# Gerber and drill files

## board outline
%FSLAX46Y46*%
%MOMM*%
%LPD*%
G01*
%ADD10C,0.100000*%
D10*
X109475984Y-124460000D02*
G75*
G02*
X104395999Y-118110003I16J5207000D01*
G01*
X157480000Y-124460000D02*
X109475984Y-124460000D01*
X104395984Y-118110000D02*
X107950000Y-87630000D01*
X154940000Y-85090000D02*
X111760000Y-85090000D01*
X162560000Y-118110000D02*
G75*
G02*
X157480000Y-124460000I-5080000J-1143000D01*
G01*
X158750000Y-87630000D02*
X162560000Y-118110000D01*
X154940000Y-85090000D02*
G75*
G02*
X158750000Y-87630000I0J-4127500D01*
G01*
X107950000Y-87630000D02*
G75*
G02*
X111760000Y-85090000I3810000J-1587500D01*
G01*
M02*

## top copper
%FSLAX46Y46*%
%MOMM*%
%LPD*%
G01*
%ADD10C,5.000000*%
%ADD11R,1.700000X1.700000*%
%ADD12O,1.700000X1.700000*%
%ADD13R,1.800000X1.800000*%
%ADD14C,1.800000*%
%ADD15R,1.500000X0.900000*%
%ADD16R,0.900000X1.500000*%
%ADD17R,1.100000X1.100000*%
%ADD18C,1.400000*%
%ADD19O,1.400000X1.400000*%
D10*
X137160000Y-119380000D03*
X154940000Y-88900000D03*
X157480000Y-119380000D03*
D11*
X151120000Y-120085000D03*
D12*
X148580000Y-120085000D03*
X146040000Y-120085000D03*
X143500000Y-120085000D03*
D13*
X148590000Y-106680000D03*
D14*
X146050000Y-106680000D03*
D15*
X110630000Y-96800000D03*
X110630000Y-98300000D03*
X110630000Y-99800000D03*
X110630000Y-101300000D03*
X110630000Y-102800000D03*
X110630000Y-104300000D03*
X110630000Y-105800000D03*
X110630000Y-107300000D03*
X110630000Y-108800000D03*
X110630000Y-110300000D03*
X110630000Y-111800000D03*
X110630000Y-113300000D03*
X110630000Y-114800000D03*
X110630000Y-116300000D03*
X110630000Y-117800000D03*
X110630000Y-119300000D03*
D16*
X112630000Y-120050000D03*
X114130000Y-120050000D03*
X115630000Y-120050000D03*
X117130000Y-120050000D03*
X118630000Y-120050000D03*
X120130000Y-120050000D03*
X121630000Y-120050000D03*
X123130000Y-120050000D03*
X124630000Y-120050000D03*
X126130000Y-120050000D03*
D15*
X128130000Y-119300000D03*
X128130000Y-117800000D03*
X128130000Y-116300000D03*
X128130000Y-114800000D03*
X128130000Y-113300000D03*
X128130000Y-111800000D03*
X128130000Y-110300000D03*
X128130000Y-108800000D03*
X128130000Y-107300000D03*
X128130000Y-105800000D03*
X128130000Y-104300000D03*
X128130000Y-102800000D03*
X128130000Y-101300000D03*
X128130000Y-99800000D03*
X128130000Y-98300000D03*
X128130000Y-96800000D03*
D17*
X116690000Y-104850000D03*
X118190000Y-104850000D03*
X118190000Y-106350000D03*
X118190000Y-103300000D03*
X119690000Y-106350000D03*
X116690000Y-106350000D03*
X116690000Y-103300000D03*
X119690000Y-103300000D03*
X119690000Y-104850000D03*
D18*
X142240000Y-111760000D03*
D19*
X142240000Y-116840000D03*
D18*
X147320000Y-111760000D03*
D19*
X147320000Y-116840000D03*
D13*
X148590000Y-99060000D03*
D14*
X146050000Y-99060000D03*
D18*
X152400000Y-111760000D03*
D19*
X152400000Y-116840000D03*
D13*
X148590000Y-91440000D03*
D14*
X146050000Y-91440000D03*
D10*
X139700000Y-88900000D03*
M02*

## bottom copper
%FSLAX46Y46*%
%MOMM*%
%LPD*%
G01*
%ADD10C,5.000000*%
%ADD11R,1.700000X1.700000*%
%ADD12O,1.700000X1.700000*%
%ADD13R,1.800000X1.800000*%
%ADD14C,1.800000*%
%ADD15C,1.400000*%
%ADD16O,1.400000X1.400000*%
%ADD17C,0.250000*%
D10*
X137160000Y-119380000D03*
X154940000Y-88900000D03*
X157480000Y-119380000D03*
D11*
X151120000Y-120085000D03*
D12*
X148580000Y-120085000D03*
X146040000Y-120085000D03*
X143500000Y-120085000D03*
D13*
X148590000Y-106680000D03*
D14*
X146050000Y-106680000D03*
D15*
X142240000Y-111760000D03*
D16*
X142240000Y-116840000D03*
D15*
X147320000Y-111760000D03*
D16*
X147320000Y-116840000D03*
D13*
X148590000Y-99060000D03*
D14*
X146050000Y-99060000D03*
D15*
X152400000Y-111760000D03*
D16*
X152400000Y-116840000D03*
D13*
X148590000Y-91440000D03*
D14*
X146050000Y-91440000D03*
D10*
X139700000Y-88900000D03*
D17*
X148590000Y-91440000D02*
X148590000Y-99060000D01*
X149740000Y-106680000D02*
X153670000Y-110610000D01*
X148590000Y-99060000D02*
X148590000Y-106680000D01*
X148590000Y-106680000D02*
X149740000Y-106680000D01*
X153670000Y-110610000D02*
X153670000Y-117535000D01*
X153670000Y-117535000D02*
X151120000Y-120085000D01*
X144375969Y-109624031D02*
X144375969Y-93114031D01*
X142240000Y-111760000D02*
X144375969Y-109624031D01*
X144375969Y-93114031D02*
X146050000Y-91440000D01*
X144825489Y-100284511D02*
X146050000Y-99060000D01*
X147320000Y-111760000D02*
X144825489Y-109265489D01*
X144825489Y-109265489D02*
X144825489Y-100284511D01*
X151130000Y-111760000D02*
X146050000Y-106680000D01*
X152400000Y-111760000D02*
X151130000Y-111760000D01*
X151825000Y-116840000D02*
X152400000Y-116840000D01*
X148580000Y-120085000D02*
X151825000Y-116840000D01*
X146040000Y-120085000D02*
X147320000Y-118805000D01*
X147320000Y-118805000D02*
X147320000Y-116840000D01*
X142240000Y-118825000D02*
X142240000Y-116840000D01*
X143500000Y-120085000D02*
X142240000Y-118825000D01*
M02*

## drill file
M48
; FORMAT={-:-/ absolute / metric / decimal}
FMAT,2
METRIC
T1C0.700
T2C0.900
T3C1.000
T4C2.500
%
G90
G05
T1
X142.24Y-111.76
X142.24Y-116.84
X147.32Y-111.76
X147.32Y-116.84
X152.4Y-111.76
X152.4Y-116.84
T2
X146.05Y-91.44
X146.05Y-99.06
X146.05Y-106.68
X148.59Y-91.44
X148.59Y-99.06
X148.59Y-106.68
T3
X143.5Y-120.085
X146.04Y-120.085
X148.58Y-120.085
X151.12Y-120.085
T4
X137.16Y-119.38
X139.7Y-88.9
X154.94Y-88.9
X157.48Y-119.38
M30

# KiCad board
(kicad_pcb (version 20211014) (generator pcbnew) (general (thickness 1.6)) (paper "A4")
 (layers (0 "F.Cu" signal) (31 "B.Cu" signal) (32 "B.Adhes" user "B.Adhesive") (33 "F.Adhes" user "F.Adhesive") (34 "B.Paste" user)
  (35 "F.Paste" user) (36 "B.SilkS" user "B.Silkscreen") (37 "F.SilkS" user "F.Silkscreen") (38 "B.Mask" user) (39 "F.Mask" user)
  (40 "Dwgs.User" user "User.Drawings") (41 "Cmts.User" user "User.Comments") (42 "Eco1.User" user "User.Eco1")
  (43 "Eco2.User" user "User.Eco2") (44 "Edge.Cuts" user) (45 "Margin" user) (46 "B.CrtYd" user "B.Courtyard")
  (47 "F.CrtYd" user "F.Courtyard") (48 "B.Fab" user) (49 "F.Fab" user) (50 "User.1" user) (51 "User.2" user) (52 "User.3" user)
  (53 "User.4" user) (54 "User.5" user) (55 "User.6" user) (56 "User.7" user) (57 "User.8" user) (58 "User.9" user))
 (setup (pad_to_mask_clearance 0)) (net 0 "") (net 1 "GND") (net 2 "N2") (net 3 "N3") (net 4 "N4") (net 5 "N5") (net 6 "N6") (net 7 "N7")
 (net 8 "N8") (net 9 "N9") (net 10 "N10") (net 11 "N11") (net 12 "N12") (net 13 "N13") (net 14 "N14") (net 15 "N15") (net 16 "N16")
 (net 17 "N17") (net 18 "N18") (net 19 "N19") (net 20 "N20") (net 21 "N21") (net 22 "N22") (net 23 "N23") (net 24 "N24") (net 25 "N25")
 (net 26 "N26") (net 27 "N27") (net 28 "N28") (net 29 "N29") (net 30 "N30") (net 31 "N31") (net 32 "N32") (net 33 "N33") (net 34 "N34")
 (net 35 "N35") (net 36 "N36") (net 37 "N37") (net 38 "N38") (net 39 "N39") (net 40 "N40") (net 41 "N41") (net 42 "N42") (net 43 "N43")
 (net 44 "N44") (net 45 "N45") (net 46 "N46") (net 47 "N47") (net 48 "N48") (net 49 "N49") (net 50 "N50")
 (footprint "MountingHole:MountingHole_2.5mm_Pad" (layer "F.Cu") (at 137.16 119.38)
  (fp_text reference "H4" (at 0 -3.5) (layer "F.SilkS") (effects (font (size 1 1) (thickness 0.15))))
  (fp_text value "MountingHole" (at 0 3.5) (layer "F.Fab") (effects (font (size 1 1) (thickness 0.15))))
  (pad "1" thru_hole circle (at 0 0) (size 5 5) (drill 2.5) (layers *.Cu *.Mask)))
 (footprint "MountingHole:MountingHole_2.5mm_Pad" (layer "F.Cu") (at 154.94 88.9 180)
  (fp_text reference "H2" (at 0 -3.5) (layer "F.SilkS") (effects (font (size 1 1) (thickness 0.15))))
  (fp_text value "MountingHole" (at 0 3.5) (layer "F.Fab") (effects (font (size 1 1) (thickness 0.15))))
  (pad "1" thru_hole circle (at 0 0 180) (size 5 5) (drill 2.5) (layers *.Cu *.Mask)))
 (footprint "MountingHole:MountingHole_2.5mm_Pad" (layer "F.Cu") (at 157.48 119.38)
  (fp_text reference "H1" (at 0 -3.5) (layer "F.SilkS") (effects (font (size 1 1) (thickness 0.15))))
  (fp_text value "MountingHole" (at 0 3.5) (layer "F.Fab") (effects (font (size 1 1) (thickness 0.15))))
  (pad "1" thru_hole circle (at 0 0) (size 5 5) (drill 2.5) (layers *.Cu *.Mask)))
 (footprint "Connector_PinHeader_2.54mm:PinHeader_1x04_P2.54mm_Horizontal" (layer "F.Cu") (at 151.12 120.085 -90)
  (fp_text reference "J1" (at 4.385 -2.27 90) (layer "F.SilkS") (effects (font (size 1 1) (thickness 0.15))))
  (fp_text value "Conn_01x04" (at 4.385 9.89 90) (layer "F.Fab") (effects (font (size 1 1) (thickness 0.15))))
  (pad "1" thru_hole rect (at 0 0 270) (size 1.7 1.7) (drill 1) (layers *.Cu *.Mask) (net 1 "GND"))
  (pad "2" thru_hole oval (at 0 2.54 270) (size 1.7 1.7) (drill 1) (layers *.Cu *.Mask) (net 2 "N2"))
  (pad "3" thru_hole oval (at 0 5.08 270) (size 1.7 1.7) (drill 1) (layers *.Cu *.Mask) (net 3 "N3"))
  (pad "4" thru_hole oval (at 0 7.62 270) (size 1.7 1.7) (drill 1) (layers *.Cu *.Mask) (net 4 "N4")))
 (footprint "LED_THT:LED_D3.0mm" (layer "F.Cu") (at 148.59 106.68 180)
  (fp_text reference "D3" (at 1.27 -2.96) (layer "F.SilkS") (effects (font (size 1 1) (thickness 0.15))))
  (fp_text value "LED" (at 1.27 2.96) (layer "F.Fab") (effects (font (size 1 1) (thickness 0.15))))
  (pad "1" thru_hole rect (at 0 0 180) (size 1.8 1.8) (drill 0.9) (layers *.Cu *.Mask) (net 1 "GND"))
  (pad "2" thru_hole circle (at 2.54 0 180) (size 1.8 1.8) (drill 0.9) (layers *.Cu *.Mask) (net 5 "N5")))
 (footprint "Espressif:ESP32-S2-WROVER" (layer "F.Cu") (at 119.38 107.95)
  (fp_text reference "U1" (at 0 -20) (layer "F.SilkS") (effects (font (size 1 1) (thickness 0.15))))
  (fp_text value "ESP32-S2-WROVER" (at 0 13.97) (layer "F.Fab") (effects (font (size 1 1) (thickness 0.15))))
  (pad "1" smd rect locked (at -8.75 -11.15) (size 1.5 0.9) (layers "F.Cu" "F.Paste" "F.Mask") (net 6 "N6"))
  (pad "2" smd rect locked (at -8.75 -9.65) (size 1.5 0.9) (layers "F.Cu" "F.Paste" "F.Mask") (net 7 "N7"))
  (pad "3" smd rect locked (at -8.75 -8.15) (size 1.5 0.9) (layers "F.Cu" "F.Paste" "F.Mask") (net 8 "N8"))
  (pad "4" smd rect locked (at -8.75 -6.65) (size 1.5 0.9) (layers "F.Cu" "F.Paste" "F.Mask") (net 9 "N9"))
  (pad "5" smd rect locked (at -8.75 -5.15) (size 1.5 0.9) (layers "F.Cu" "F.Paste" "F.Mask") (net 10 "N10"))
  (pad "6" smd rect locked (at -8.75 -3.65) (size 1.5 0.9) (layers "F.Cu" "F.Paste" "F.Mask") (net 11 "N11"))
  (pad "7" smd rect locked (at -8.75 -2.15) (size 1.5 0.9) (layers "F.Cu" "F.Paste" "F.Mask") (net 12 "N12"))
  (pad "8" smd rect locked (at -8.75 -0.65) (size 1.5 0.9) (layers "F.Cu" "F.Paste" "F.Mask") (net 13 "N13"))
  (pad "9" smd rect locked (at -8.75 0.85) (size 1.5 0.9) (layers "F.Cu" "F.Paste" "F.Mask") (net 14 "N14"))
  (pad "10" smd rect locked (at -8.75 2.35) (size 1.5 0.9) (layers "F.Cu" "F.Paste" "F.Mask") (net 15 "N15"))
  (pad "11" smd rect locked (at -8.75 3.85) (size 1.5 0.9) (layers "F.Cu" "F.Paste" "F.Mask") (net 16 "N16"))
  (pad "12" smd rect locked (at -8.75 5.35) (size 1.5 0.9) (layers "F.Cu" "F.Paste" "F.Mask") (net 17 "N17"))
  (pad "13" smd rect locked (at -8.75 6.85) (size 1.5 0.9) (layers "F.Cu" "F.Paste" "F.Mask") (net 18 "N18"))
  (pad "14" smd rect locked (at -8.75 8.35) (size 1.5 0.9) (layers "F.Cu" "F.Paste" "F.Mask") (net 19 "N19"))
  (pad "15" smd rect locked (at -8.75 9.85) (size 1.5 0.9) (layers "F.Cu" "F.Paste" "F.Mask") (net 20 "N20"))
  (pad "16" smd rect locked (at -8.75 11.35) (size 1.5 0.9) (layers "F.Cu" "F.Paste" "F.Mask") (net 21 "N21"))
  (pad "17" smd rect locked (at -6.75 12.1 90) (size 1.5 0.9) (layers "F.Cu" "F.Paste" "F.Mask") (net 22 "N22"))
  (pad "18" smd rect locked (at -5.25 12.1 90) (size 1.5 0.9) (layers "F.Cu" "F.Paste" "F.Mask") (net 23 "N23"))
  (pad "19" smd rect locked (at -3.75 12.1 90) (size 1.5 0.9) (layers "F.Cu" "F.Paste" "F.Mask") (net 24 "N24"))
  (pad "20" smd rect locked (at -2.25 12.1 90) (size 1.5 0.9) (layers "F.Cu" "F.Paste" "F.Mask") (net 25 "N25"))
  (pad "21" smd rect locked (at -0.75 12.1 90) (size 1.5 0.9) (layers "F.Cu" "F.Paste" "F.Mask") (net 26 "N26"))
  (pad "22" smd rect locked (at 0.75 12.1 90) (size 1.5 0.9) (layers "F.Cu" "F.Paste" "F.Mask") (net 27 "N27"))
  (pad "23" smd rect locked (at 2.25 12.1 90) (size 1.5 0.9) (layers "F.Cu" "F.Paste" "F.Mask") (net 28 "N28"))
  (pad "24" smd rect locked (at 3.75 12.1 90) (size 1.5 0.9) (layers "F.Cu" "F.Paste" "F.Mask") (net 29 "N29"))
  (pad "25" smd rect locked (at 5.25 12.1 90) (size 1.5 0.9) (layers "F.Cu" "F.Paste" "F.Mask") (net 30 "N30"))
  (pad "26" smd rect locked (at 6.75 12.1 90) (size 1.5 0.9) (layers "F.Cu" "F.Paste" "F.Mask") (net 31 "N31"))
  (pad "27" smd rect locked (at 8.75 11.35 180) (size 1.5 0.9) (layers "F.Cu" "F.Paste" "F.Mask") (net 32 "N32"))
  (pad "28" smd rect locked (at 8.75 9.85 180) (size 1.5 0.9) (layers "F.Cu" "F.Paste" "F.Mask") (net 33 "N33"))
  (pad "29" smd rect locked (at 8.75 8.35 180) (size 1.5 0.9) (layers "F.Cu" "F.Paste" "F.Mask") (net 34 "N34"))
  (pad "30" smd rect locked (at 8.75 6.85 180) (size 1.5 0.9) (layers "F.Cu" "F.Paste" "F.Mask") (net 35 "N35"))
  (pad "31" smd rect locked (at 8.75 5.35 180) (size 1.5 0.9) (layers "F.Cu" "F.Paste" "F.Mask") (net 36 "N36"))
  (pad "32" smd rect locked (at 8.75 3.85 180) (size 1.5 0.9) (layers "F.Cu" "F.Paste" "F.Mask") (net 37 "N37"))
  (pad "33" smd rect locked (at 8.75 2.35 180) (size 1.5 0.9) (layers "F.Cu" "F.Paste" "F.Mask") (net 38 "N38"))
  (pad "34" smd rect locked (at 8.75 0.85 180) (size 1.5 0.9) (layers "F.Cu" "F.Paste" "F.Mask") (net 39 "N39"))
  (pad "35" smd rect locked (at 8.75 -0.65 180) (size 1.5 0.9) (layers "F.Cu" "F.Paste" "F.Mask") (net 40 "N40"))
  (pad "36" smd rect locked (at 8.75 -2.15 180) (size 1.5 0.9) (layers "F.Cu" "F.Paste" "F.Mask") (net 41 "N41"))
  (pad "37" smd rect locked (at 8.75 -3.65 180) (size 1.5 0.9) (layers "F.Cu" "F.Paste" "F.Mask") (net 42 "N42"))
  (pad "38" smd rect locked (at 8.75 -5.15 180) (size 1.5 0.9) (layers "F.Cu" "F.Paste" "F.Mask") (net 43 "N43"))
  (pad "39" smd rect locked (at 8.75 -6.65 180) (size 1.5 0.9) (layers "F.Cu" "F.Paste" "F.Mask") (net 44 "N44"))
  (pad "40" smd rect locked (at 8.75 -8.15 180) (size 1.5 0.9) (layers "F.Cu" "F.Paste" "F.Mask") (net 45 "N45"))
  (pad "41" smd rect locked (at 8.75 -9.65 180) (size 1.5 0.9) (layers "F.Cu" "F.Paste" "F.Mask") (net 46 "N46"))
  (pad "42" smd rect locked (at 8.75 -11.15 180) (size 1.5 0.9) (layers "F.Cu" "F.Paste" "F.Mask") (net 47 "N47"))
  (pad "43" smd rect locked (at -2.69 -3.1 180) (size 1.1 1.1) (layers "F.Cu" "F.Paste" "F.Mask") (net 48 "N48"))
  (pad "43" smd rect locked (at -1.19 -3.1 180) (size 1.1 1.1) (layers "F.Cu" "F.Paste" "F.Mask") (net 48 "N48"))
  (pad "43" smd rect locked (at -1.19 -1.6 180) (size 1.1 1.1) (layers "F.Cu" "F.Paste" "F.Mask") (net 48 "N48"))
  (pad "43" smd rect locked (at -1.19 -4.65 180) (size 1.1 1.1) (layers "F.Cu" "F.Paste" "F.Mask") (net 48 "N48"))
  (pad "43" smd rect locked (at 0.31 -1.6 180) (size 1.1 1.1) (layers "F.Cu" "F.Paste" "F.Mask") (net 48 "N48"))
  (pad "43" smd rect locked (at -2.69 -1.6 180) (size 1.1 1.1) (layers "F.Cu" "F.Paste" "F.Mask") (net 48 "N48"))
  (pad "43" smd rect locked (at -2.69 -4.65 180) (size 1.1 1.1) (layers "F.Cu" "F.Paste" "F.Mask") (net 48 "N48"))
  (pad "43" smd rect locked (at 0.31 -4.65 180) (size 1.1 1.1) (layers "F.Cu" "F.Paste" "F.Mask") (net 48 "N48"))
  (pad "43" smd rect locked (at 0.31 -3.1 180) (size 1.1 1.1) (layers "F.Cu" "F.Paste" "F.Mask") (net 48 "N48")))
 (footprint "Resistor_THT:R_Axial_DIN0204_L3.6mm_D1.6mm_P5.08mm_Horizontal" (layer "F.Cu") (at 142.24 111.76 -90)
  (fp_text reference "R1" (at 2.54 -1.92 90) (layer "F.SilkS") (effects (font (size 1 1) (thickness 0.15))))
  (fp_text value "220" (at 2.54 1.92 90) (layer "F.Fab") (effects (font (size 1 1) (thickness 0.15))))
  (pad "1" thru_hole circle (at 0 0 270) (size 1.4 1.4) (drill 0.7) (layers *.Cu *.Mask) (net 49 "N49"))
  (pad "2" thru_hole oval (at 5.08 0 270) (size 1.4 1.4) (drill 0.7) (layers *.Cu *.Mask) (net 4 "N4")))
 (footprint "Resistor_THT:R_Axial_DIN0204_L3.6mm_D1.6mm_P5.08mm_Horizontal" (layer "F.Cu") (at 147.32 111.76 -90)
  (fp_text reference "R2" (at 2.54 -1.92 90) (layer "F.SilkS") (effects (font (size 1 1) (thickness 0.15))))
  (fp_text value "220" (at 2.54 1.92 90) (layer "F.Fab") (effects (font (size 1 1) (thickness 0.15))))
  (pad "1" thru_hole circle (at 0 0 270) (size 1.4 1.4) (drill 0.7) (layers *.Cu *.Mask) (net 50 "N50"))
  (pad "2" thru_hole oval (at 5.08 0 270) (size 1.4 1.4) (drill 0.7) (layers *.Cu *.Mask) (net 3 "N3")))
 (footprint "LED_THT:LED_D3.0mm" (layer "F.Cu") (at 148.59 99.06 180)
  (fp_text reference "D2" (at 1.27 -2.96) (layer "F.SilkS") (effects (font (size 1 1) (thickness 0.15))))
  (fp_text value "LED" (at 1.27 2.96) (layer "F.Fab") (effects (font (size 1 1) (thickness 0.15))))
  (pad "1" thru_hole rect (at 0 0 180) (size 1.8 1.8) (drill 0.9) (layers *.Cu *.Mask) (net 1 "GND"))
  (pad "2" thru_hole circle (at 2.54 0 180) (size 1.8 1.8) (drill 0.9) (layers *.Cu *.Mask) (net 50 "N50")))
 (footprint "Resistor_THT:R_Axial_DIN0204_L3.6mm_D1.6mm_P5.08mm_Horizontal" (layer "F.Cu") (at 152.4 111.76 -90)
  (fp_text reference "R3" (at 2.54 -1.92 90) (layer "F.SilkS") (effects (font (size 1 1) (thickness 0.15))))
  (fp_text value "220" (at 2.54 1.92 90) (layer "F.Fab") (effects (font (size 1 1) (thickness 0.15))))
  (pad "1" thru_hole circle (at 0 0 270) (size 1.4 1.4) (drill 0.7) (layers *.Cu *.Mask) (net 5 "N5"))
  (pad "2" thru_hole oval (at 5.08 0 270) (size 1.4 1.4) (drill 0.7) (layers *.Cu *.Mask) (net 2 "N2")))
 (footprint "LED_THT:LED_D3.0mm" (layer "F.Cu") (at 148.59 91.44 180)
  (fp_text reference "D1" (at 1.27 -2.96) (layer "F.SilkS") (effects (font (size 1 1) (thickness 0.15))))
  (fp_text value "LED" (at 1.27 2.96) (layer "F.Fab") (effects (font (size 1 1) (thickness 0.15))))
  (pad "1" thru_hole rect (at 0 0 180) (size 1.8 1.8) (drill 0.9) (layers *.Cu *.Mask) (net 1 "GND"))
  (pad "2" thru_hole circle (at 2.54 0 180) (size 1.8 1.8) (drill 0.9) (layers *.Cu *.Mask) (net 49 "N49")))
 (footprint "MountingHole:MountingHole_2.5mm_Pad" (layer "F.Cu") (at 139.7 88.9 180)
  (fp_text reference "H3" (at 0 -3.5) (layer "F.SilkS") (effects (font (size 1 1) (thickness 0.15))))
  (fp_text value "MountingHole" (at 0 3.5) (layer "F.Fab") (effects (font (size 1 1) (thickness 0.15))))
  (pad "1" thru_hole circle (at 0 0 180) (size 5 5) (drill 2.5) (layers *.Cu *.Mask)))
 (gr_arc (start 109.475984 124.46) (mid 105.41 122.505787) (end 104.395984 118.11) (layer "Edge.Cuts") (width 0.1))
 (gr_line (start 157.48 124.46) (end 109.475984 124.46) (layer "Edge.Cuts") (width 0.1))
 (gr_line (start 104.395984 118.11) (end 107.95 87.63) (layer "Edge.Cuts") (width 0.1))
 (gr_line (start 154.94 85.09) (end 111.76 85.09) (layer "Edge.Cuts") (width 0.1))
 (gr_arc (start 162.56 118.11) (mid 161.545984 122.505787) (end 157.48 124.46) (layer "Edge.Cuts") (width 0.1))
 (gr_line (start 158.75 87.63) (end 162.56 118.11) (layer "Edge.Cuts") (width 0.1))
 (gr_arc (start 154.94 85.09) (mid 157.229525 85.783212) (end 158.75 87.63) (layer "Edge.Cuts") (width 0.1))
 (gr_arc (start 107.95 87.63) (mid 109.470475 85.783212) (end 111.76 85.09) (layer "Edge.Cuts") (width 0.1))
 (segment (start 148.59 91.44) (end 148.59 99.06) (width 0.25) (layer "B.Cu") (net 1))
 (segment (start 149.74 106.68) (end 153.67 110.61) (width 0.25) (layer "B.Cu") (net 1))
 (segment (start 148.59 99.06) (end 148.59 106.68) (width 0.25) (layer "B.Cu") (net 1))
 (segment (start 148.59 106.68) (end 149.74 106.68) (width 0.25) (layer "B.Cu") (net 1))
 (segment (start 153.67 110.61) (end 153.67 117.535) (width 0.25) (layer "B.Cu") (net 1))
 (segment (start 153.67 117.535) (end 151.12 120.085) (width 0.25) (layer "B.Cu") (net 1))
 (segment (start 144.375969 109.624031) (end 144.375969 93.114031) (width 0.25) (layer "B.Cu") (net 49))
 (segment (start 142.24 111.76) (end 144.375969 109.624031) (width 0.25) (layer "B.Cu") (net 49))
 (segment (start 144.375969 93.114031) (end 146.05 91.44) (width 0.25) (layer "B.Cu") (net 49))
 (segment (start 144.825489 100.284511) (end 146.05 99.06) (width 0.25) (layer "B.Cu") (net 50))
 (segment (start 147.32 111.76) (end 144.825489 109.265489) (width 0.25) (layer "B.Cu") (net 50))
 (segment (start 144.825489 109.265489) (end 144.825489 100.284511) (width 0.25) (layer "B.Cu") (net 50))
 (segment (start 151.13 111.76) (end 146.05 106.68) (width 0.25) (layer "B.Cu") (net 5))
 (segment (start 152.4 111.76) (end 151.13 111.76) (width 0.25) (layer "B.Cu") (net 5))
 (segment (start 151.825 116.84) (end 152.4 116.84) (width 0.25) (layer "B.Cu") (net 2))
 (segment (start 148.58 120.085) (end 151.825 116.84) (width 0.25) (layer "B.Cu") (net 2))
 (segment (start 146.04 120.085) (end 147.32 118.805) (width 0.25) (layer "B.Cu") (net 3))
 (segment (start 147.32 118.805) (end 147.32 116.84) (width 0.25) (layer "B.Cu") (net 3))
 (segment (start 142.24 118.825) (end 142.24 116.84) (width 0.25) (layer "B.Cu") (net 4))
 (segment (start 143.5 120.085) (end 142.24 118.825) (width 0.25) (layer "B.Cu") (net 4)))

